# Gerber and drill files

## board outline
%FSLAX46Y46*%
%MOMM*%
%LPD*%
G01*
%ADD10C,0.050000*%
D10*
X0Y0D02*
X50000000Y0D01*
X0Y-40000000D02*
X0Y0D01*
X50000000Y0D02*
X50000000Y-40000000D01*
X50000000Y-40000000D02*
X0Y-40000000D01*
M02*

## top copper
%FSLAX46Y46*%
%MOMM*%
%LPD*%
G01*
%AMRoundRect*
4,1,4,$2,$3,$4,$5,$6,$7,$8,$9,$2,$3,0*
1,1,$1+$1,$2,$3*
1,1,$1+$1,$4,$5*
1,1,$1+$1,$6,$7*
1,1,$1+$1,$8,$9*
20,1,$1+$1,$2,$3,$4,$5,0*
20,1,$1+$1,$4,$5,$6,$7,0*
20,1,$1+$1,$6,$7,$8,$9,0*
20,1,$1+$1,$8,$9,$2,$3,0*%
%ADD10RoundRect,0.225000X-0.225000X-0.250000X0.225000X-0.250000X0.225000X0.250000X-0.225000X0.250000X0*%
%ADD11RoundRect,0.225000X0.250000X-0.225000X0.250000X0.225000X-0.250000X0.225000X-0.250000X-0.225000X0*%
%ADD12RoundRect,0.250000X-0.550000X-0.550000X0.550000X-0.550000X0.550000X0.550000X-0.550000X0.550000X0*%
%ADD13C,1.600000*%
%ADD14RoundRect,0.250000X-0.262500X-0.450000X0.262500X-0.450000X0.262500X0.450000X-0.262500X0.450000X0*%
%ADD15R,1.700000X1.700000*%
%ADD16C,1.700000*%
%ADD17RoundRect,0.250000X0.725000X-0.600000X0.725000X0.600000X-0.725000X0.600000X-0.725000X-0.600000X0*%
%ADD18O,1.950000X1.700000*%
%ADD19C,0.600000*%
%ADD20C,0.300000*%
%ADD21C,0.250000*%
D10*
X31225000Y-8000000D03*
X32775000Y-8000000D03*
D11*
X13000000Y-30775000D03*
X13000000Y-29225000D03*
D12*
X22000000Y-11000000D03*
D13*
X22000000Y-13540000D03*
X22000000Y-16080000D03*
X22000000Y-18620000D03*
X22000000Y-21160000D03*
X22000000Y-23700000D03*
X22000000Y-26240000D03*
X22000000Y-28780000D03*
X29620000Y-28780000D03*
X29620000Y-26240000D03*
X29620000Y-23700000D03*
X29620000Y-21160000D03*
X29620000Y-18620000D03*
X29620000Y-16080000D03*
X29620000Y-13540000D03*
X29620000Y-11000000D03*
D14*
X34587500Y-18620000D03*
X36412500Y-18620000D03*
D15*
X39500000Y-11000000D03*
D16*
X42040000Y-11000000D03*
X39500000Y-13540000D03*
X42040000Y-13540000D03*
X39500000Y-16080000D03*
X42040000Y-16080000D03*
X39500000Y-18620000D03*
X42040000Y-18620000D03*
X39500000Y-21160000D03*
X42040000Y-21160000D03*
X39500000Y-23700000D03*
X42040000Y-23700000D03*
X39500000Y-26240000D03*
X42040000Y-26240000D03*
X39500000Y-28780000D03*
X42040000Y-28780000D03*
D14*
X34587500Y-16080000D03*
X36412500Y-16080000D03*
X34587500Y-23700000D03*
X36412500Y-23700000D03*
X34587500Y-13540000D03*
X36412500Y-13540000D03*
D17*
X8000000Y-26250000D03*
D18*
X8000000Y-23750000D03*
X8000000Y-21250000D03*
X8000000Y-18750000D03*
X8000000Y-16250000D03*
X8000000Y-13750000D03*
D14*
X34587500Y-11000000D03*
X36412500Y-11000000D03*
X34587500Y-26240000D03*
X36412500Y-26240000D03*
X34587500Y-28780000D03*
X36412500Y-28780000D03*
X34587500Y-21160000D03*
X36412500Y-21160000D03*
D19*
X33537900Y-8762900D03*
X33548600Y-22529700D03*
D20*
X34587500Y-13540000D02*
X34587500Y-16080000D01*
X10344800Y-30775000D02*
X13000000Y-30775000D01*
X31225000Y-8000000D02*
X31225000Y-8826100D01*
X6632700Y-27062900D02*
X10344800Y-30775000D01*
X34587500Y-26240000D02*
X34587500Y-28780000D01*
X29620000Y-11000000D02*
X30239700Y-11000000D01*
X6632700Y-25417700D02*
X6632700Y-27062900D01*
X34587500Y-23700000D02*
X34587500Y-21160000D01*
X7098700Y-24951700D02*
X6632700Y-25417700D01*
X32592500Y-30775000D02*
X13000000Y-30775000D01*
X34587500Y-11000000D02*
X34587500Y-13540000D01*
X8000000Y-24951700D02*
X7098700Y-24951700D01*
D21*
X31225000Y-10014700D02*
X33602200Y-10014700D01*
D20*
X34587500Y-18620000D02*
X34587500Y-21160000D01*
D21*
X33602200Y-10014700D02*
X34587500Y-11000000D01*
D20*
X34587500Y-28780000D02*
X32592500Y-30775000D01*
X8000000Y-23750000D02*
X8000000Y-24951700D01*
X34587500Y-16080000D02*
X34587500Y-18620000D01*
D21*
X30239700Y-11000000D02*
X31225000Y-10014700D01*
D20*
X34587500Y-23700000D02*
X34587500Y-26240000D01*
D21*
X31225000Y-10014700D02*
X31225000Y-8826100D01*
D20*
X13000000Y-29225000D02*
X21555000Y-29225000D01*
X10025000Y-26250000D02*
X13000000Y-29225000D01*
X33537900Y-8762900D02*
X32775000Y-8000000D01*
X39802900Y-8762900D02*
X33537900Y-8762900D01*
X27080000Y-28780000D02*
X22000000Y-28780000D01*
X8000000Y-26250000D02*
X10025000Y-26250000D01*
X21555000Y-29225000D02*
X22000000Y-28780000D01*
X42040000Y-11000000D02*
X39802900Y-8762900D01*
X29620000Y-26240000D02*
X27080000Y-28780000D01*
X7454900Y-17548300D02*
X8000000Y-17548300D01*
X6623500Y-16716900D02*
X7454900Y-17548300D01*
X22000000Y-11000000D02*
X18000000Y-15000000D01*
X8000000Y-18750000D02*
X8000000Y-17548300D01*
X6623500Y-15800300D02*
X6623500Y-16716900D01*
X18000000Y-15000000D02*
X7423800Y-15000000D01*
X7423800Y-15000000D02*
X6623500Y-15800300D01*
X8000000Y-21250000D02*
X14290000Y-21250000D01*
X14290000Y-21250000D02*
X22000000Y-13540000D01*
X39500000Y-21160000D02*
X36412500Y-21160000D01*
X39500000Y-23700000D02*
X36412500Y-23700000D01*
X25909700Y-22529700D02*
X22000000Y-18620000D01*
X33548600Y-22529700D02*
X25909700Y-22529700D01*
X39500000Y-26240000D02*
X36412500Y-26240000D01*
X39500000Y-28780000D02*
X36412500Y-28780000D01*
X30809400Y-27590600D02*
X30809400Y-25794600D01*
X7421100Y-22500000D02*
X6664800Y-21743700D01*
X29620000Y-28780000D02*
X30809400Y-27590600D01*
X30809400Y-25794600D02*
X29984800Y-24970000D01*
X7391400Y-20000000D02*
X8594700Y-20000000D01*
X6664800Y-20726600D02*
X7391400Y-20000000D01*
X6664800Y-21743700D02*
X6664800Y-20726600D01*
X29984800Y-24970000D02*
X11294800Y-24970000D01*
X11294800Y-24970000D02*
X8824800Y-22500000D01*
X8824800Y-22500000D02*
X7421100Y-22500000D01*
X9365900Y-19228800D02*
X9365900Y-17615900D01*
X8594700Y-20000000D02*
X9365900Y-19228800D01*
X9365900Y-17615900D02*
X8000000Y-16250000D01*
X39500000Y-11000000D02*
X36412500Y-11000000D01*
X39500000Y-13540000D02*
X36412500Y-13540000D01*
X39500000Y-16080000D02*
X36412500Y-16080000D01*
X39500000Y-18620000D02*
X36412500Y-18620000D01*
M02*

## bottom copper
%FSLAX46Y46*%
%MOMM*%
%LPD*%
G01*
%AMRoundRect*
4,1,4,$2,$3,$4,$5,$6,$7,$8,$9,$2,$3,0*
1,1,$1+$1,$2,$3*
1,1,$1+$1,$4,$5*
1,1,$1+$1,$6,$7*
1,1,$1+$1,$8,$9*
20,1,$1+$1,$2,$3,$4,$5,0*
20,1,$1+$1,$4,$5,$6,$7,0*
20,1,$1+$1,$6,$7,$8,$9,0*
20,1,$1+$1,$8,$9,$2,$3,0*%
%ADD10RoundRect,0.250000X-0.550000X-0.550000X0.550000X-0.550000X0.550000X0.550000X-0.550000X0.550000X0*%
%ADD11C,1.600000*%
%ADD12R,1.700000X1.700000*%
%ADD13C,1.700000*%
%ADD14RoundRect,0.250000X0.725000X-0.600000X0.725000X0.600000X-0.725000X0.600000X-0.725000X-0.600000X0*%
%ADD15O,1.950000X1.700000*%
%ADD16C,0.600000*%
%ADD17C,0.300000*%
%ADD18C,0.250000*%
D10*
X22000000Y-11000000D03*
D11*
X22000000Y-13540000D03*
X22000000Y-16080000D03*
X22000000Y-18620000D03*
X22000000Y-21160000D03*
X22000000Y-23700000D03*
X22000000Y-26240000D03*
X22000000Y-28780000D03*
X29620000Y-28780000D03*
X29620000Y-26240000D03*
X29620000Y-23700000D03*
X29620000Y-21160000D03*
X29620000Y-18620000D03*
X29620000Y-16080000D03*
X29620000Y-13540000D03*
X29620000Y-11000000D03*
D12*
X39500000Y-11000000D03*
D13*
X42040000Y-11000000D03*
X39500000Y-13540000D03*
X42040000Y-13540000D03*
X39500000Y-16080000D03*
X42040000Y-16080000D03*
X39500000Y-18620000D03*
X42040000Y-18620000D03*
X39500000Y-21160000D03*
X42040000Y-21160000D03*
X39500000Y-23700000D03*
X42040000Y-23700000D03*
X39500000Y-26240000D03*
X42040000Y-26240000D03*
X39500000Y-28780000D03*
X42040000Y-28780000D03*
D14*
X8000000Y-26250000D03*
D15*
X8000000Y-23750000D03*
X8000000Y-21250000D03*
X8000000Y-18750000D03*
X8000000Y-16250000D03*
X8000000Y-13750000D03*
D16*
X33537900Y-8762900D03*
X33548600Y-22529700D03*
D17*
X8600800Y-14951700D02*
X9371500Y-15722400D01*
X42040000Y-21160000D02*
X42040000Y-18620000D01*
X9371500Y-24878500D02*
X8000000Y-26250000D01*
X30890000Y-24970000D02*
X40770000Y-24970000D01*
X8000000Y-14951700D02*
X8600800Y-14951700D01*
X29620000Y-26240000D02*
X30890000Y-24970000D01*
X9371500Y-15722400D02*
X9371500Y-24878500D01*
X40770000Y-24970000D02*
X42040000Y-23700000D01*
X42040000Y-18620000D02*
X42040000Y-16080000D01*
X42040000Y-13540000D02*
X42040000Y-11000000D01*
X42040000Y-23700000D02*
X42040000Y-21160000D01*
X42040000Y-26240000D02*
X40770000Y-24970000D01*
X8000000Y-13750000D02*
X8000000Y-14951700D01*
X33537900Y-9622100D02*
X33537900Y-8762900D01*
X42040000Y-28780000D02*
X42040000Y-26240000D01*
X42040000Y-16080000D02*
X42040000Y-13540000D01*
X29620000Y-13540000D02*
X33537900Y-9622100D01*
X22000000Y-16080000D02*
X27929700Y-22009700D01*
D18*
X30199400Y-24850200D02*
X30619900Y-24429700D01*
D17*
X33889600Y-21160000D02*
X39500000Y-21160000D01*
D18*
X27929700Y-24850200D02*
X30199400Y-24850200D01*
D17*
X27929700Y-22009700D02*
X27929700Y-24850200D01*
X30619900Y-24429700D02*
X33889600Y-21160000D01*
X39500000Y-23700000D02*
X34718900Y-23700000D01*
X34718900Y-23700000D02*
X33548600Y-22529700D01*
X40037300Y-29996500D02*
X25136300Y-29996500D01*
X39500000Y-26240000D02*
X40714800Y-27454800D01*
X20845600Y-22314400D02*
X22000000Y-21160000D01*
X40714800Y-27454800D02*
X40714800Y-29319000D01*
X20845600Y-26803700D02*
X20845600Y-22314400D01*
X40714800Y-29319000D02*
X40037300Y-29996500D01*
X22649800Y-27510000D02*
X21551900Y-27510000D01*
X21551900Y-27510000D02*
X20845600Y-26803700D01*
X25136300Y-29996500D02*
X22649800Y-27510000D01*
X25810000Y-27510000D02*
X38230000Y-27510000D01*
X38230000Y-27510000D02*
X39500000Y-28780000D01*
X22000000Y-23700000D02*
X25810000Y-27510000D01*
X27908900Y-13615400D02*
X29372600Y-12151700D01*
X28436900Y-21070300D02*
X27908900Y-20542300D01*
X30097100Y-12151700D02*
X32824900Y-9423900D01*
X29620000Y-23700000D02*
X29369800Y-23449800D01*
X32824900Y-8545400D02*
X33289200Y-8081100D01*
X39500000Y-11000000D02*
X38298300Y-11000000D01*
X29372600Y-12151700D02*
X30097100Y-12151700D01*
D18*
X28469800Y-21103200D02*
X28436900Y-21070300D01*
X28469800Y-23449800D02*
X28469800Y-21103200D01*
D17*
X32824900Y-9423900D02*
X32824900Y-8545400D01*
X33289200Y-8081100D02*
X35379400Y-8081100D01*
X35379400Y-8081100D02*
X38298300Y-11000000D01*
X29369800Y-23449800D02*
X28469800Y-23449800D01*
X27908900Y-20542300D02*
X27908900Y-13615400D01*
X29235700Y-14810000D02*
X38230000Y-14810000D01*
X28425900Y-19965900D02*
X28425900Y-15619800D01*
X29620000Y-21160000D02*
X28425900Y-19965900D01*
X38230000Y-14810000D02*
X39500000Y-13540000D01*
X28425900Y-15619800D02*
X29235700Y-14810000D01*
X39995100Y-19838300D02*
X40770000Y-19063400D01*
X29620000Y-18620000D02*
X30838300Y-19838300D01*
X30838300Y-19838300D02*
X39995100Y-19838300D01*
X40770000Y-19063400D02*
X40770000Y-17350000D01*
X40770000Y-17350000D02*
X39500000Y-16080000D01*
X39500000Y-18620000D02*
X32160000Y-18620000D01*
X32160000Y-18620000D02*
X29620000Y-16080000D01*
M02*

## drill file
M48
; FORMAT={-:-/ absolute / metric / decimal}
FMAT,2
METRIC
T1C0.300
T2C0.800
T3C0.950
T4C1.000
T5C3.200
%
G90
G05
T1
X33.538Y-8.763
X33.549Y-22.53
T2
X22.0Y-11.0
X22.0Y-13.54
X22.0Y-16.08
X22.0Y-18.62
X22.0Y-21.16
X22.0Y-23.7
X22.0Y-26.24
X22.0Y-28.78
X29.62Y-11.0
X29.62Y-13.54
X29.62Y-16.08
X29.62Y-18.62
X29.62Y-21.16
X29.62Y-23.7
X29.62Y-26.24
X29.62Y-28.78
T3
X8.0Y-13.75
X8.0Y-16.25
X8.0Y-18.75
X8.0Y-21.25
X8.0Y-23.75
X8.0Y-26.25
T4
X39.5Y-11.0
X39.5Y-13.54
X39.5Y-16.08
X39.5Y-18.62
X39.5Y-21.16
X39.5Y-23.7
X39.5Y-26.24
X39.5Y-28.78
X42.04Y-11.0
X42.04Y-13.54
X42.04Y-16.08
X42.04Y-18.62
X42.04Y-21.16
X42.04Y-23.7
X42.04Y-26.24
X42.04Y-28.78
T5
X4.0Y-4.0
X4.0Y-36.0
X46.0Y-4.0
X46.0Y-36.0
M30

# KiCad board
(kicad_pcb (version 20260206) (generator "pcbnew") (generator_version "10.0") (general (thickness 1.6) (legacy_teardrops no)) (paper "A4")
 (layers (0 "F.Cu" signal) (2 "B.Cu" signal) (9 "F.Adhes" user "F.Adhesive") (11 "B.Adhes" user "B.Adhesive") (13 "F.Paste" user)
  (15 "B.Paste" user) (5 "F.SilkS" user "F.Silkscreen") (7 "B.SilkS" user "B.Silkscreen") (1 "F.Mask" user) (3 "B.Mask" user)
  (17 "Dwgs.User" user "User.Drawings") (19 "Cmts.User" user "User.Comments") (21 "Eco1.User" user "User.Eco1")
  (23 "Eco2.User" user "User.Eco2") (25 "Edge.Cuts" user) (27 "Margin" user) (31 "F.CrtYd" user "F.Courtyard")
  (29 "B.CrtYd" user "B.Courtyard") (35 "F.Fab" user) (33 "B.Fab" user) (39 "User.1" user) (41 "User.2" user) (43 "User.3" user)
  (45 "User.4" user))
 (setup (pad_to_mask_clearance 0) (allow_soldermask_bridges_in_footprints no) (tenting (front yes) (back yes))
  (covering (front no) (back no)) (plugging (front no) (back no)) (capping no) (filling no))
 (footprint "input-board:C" (layer "F.Cu") (at 32 8)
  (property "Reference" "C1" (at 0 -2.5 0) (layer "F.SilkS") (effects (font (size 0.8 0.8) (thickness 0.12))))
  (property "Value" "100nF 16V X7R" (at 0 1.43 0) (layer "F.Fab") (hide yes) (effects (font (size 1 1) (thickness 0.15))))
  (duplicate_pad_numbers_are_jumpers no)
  (pad "1" smd roundrect (at -0.775 0) (size 0.9 0.95) (layers "F.Cu" "F.Mask" "F.Paste") (roundrect_rratio 0.25) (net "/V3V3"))
  (pad "2" smd roundrect (at 0.775 0) (size 0.9 0.95) (layers "F.Cu" "F.Mask" "F.Paste") (roundrect_rratio 0.25) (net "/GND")))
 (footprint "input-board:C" (layer "F.Cu") (at 13 30 90)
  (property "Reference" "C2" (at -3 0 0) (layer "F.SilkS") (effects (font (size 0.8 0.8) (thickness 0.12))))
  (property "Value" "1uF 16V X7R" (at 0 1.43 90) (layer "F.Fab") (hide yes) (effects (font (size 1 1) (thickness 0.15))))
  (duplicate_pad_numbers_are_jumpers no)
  (pad "1" smd roundrect (at -0.775 0 90) (size 0.9 0.95) (layers "F.Cu" "F.Mask" "F.Paste") (roundrect_rratio 0.25) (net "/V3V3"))
  (pad "2" smd roundrect (at 0.775 0 90) (size 0.9 0.95) (layers "F.Cu" "F.Mask" "F.Paste") (roundrect_rratio 0.25) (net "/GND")))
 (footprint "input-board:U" (layer "F.Cu") (at 22 11)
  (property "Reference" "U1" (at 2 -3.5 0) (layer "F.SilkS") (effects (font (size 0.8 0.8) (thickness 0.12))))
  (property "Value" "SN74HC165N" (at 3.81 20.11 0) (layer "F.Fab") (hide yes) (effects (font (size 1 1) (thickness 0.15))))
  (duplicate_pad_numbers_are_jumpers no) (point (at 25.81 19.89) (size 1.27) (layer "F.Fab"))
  (pad "1" thru_hole roundrect (at 0 0) (size 1.6 1.6) (drill 0.8) (layers "*.Cu" "*.Mask") (remove_unused_layers no)
   (roundrect_rratio 0.15625) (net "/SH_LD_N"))
  (pad "2" thru_hole circle (at 0 2.54) (size 1.6 1.6) (drill 0.8) (layers "*.Cu" "*.Mask") (remove_unused_layers no) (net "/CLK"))
  (pad "3" thru_hole circle (at 0 5.08) (size 1.6 1.6) (drill 0.8) (layers "*.Cu" "*.Mask") (remove_unused_layers no) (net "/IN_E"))
  (pad "4" thru_hole circle (at 0 7.62) (size 1.6 1.6) (drill 0.8) (layers "*.Cu" "*.Mask") (remove_unused_layers no) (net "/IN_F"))
  (pad "5" thru_hole circle (at 0 10.16) (size 1.6 1.6) (drill 0.8) (layers "*.Cu" "*.Mask") (remove_unused_layers no) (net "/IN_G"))
  (pad "6" thru_hole circle (at 0 12.7) (size 1.6 1.6) (drill 0.8) (layers "*.Cu" "*.Mask") (remove_unused_layers no) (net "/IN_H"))
  (pad "7" thru_hole circle (at 0 15.24) (size 1.6 1.6) (drill 0.8) (layers "*.Cu" "*.Mask") (remove_unused_layers no)
   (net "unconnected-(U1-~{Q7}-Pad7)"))
  (pad "8" thru_hole circle (at 0 17.78) (size 1.6 1.6) (drill 0.8) (layers "*.Cu" "*.Mask") (remove_unused_layers no) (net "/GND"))
  (pad "9" thru_hole circle (at 7.62 17.78) (size 1.6 1.6) (drill 0.8) (layers "*.Cu" "*.Mask") (remove_unused_layers no) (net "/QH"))
  (pad "10" thru_hole circle (at 7.62 15.24) (size 1.6 1.6) (drill 0.8) (layers "*.Cu" "*.Mask") (remove_unused_layers no) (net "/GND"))
  (pad "11" thru_hole circle (at 7.62 12.7) (size 1.6 1.6) (drill 0.8) (layers "*.Cu" "*.Mask") (remove_unused_layers no) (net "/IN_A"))
  (pad "12" thru_hole circle (at 7.62 10.16) (size 1.6 1.6) (drill 0.8) (layers "*.Cu" "*.Mask") (remove_unused_layers no) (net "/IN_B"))
  (pad "13" thru_hole circle (at 7.62 7.62) (size 1.6 1.6) (drill 0.8) (layers "*.Cu" "*.Mask") (remove_unused_layers no) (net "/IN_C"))
  (pad "14" thru_hole circle (at 7.62 5.08) (size 1.6 1.6) (drill 0.8) (layers "*.Cu" "*.Mask") (remove_unused_layers no) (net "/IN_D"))
  (pad "15" thru_hole circle (at 7.62 2.54) (size 1.6 1.6) (drill 0.8) (layers "*.Cu" "*.Mask") (remove_unused_layers no) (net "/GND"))
  (pad "16" thru_hole circle (at 7.62 0) (size 1.6 1.6) (drill 0.8) (layers "*.Cu" "*.Mask") (remove_unused_layers no) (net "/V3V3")))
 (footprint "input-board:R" (layer "F.Cu") (at 35.5 18.62)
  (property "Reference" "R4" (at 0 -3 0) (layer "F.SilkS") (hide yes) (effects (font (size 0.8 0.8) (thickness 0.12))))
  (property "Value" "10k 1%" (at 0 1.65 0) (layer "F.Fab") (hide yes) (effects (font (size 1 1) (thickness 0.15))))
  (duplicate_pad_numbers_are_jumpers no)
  (pad "1" smd roundrect (at -0.9125 0) (size 1.025 1.4) (layers "F.Cu" "F.Mask" "F.Paste") (roundrect_rratio 0.243902) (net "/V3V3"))
  (pad "2" smd roundrect (at 0.9125 0) (size 1.025 1.4) (layers "F.Cu" "F.Mask" "F.Paste") (roundrect_rratio 0.243902) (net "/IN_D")))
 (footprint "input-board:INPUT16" (layer "F.Cu") (at 39.5 11)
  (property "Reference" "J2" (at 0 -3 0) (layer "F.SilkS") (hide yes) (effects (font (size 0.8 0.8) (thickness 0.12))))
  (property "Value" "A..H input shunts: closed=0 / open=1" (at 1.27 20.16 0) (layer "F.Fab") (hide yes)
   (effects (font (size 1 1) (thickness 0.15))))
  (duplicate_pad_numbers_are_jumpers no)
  (pad "1" thru_hole rect (at 0 0) (size 1.7 1.7) (drill 1) (layers "*.Cu" "*.Mask") (remove_unused_layers no) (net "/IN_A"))
  (pad "2" thru_hole circle (at 2.54 0) (size 1.7 1.7) (drill 1) (layers "*.Cu" "*.Mask") (remove_unused_layers no) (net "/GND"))
  (pad "3" thru_hole circle (at 0 2.54) (size 1.7 1.7) (drill 1) (layers "*.Cu" "*.Mask") (remove_unused_layers no) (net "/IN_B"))
  (pad "4" thru_hole circle (at 2.54 2.54) (size 1.7 1.7) (drill 1) (layers "*.Cu" "*.Mask") (remove_unused_layers no) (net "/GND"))
  (pad "5" thru_hole circle (at 0 5.08) (size 1.7 1.7) (drill 1) (layers "*.Cu" "*.Mask") (remove_unused_layers no) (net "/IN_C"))
  (pad "6" thru_hole circle (at 2.54 5.08) (size 1.7 1.7) (drill 1) (layers "*.Cu" "*.Mask") (remove_unused_layers no) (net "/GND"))
  (pad "7" thru_hole circle (at 0 7.62) (size 1.7 1.7) (drill 1) (layers "*.Cu" "*.Mask") (remove_unused_layers no) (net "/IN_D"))
  (pad "8" thru_hole circle (at 2.54 7.62) (size 1.7 1.7) (drill 1) (layers "*.Cu" "*.Mask") (remove_unused_layers no) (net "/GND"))
  (pad "9" thru_hole circle (at 0 10.16) (size 1.7 1.7) (drill 1) (layers "*.Cu" "*.Mask") (remove_unused_layers no) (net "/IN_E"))
  (pad "10" thru_hole circle (at 2.54 10.16) (size 1.7 1.7) (drill 1) (layers "*.Cu" "*.Mask") (remove_unused_layers no) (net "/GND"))
  (pad "11" thru_hole circle (at 0 12.7) (size 1.7 1.7) (drill 1) (layers "*.Cu" "*.Mask") (remove_unused_layers no) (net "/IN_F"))
  (pad "12" thru_hole circle (at 2.54 12.7) (size 1.7 1.7) (drill 1) (layers "*.Cu" "*.Mask") (remove_unused_layers no) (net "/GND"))
  (pad "13" thru_hole circle (at 0 15.24) (size 1.7 1.7) (drill 1) (layers "*.Cu" "*.Mask") (remove_unused_layers no) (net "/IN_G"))
  (pad "14" thru_hole circle (at 2.54 15.24) (size 1.7 1.7) (drill 1) (layers "*.Cu" "*.Mask") (remove_unused_layers no) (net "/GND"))
  (pad "15" thru_hole circle (at 0 17.78) (size 1.7 1.7) (drill 1) (layers "*.Cu" "*.Mask") (remove_unused_layers no) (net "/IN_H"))
  (pad "16" thru_hole circle (at 2.54 17.78) (size 1.7 1.7) (drill 1) (layers "*.Cu" "*.Mask") (remove_unused_layers no) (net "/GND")))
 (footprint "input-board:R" (layer "F.Cu") (at 35.5 16.08)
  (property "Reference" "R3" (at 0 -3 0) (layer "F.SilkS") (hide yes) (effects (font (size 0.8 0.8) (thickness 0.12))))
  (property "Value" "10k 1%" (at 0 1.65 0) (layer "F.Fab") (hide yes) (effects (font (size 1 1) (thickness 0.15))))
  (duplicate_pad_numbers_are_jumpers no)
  (pad "1" smd roundrect (at -0.9125 0) (size 1.025 1.4) (layers "F.Cu" "F.Mask" "F.Paste") (roundrect_rratio 0.243902) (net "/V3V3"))
  (pad "2" smd roundrect (at 0.9125 0) (size 1.025 1.4) (layers "F.Cu" "F.Mask" "F.Paste") (roundrect_rratio 0.243902) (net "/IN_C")))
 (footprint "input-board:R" (layer "F.Cu") (at 35.5 23.7)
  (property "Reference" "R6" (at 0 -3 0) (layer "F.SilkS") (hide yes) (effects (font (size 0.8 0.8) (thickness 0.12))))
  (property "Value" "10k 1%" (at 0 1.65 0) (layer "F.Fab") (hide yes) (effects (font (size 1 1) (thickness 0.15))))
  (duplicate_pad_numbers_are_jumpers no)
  (pad "1" smd roundrect (at -0.9125 0) (size 1.025 1.4) (layers "F.Cu" "F.Mask" "F.Paste") (roundrect_rratio 0.243902) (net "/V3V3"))
  (pad "2" smd roundrect (at 0.9125 0) (size 1.025 1.4) (layers "F.Cu" "F.Mask" "F.Paste") (roundrect_rratio 0.243902) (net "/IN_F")))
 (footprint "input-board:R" (layer "F.Cu") (at 35.5 13.54)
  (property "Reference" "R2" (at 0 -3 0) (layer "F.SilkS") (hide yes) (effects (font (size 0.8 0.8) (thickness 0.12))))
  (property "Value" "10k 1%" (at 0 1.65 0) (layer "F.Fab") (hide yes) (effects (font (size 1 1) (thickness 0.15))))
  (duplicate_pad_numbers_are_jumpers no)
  (pad "1" smd roundrect (at -0.9125 0) (size 1.025 1.4) (layers "F.Cu" "F.Mask" "F.Paste") (roundrect_rratio 0.243902) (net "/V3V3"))
  (pad "2" smd roundrect (at 0.9125 0) (size 1.025 1.4) (layers "F.Cu" "F.Mask" "F.Paste") (roundrect_rratio 0.243902) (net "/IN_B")))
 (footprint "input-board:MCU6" (layer "F.Cu") (at 8 26.25 90)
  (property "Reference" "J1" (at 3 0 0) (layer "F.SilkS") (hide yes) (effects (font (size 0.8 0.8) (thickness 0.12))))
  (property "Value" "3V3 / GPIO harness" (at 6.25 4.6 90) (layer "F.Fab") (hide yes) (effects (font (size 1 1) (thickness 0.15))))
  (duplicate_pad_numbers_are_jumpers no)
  (pad "1" thru_hole roundrect (at 0 0 90) (size 1.7 1.95) (drill 0.95) (layers "*.Cu" "*.Mask") (remove_unused_layers no)
   (roundrect_rratio 0.147059) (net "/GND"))
  (pad "2" thru_hole oval (at 2.5 0 90) (size 1.7 1.95) (drill 0.95) (layers "*.Cu" "*.Mask") (remove_unused_layers no) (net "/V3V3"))
  (pad "3" thru_hole oval (at 5 0 90) (size 1.7 1.95) (drill 0.95) (layers "*.Cu" "*.Mask") (remove_unused_layers no) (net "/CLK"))
  (pad "4" thru_hole oval (at 7.5 0 90) (size 1.7 1.95) (drill 0.95) (layers "*.Cu" "*.Mask") (remove_unused_layers no) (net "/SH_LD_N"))
  (pad "5" thru_hole oval (at 10 0 90) (size 1.7 1.95) (drill 0.95) (layers "*.Cu" "*.Mask") (remove_unused_layers no) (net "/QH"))
  (pad "6" thru_hole oval (at 12.5 0 90) (size 1.7 1.95) (drill 0.95) (layers "*.Cu" "*.Mask") (remove_unused_layers no) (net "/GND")))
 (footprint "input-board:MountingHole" (layer "F.Cu") (at 4 36)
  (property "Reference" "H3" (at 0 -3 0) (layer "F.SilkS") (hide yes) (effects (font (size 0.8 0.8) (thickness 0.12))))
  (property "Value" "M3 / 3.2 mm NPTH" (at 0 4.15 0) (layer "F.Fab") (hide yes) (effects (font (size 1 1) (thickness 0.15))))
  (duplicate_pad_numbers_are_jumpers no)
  (pad "" np_thru_hole circle (at 0 0) (size 3.2 3.2) (drill 3.2) (layers "*.Cu" "*.Mask")))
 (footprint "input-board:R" (layer "F.Cu") (at 35.5 11)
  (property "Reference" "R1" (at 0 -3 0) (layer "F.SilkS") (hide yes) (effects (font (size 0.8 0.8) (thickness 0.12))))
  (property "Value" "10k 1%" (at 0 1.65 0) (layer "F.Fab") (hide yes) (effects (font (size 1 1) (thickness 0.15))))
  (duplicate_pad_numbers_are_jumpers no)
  (pad "1" smd roundrect (at -0.9125 0) (size 1.025 1.4) (layers "F.Cu" "F.Mask" "F.Paste") (roundrect_rratio 0.243902) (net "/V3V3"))
  (pad "2" smd roundrect (at 0.9125 0) (size 1.025 1.4) (layers "F.Cu" "F.Mask" "F.Paste") (roundrect_rratio 0.243902) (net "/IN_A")))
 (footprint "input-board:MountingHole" (layer "F.Cu") (at 4 4)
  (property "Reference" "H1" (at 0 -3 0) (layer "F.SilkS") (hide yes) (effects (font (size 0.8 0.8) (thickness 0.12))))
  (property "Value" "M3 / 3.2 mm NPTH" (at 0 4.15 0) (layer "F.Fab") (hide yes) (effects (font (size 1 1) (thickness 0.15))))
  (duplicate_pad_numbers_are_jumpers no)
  (pad "" np_thru_hole circle (at 0 0) (size 3.2 3.2) (drill 3.2) (layers "*.Cu" "*.Mask")))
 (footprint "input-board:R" (layer "F.Cu") (at 35.5 26.24)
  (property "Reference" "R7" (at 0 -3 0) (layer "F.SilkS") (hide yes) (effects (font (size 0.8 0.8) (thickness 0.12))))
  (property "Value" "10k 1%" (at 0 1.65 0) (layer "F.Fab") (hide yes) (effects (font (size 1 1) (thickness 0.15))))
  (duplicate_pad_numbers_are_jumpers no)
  (pad "1" smd roundrect (at -0.9125 0) (size 1.025 1.4) (layers "F.Cu" "F.Mask" "F.Paste") (roundrect_rratio 0.243902) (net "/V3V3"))
  (pad "2" smd roundrect (at 0.9125 0) (size 1.025 1.4) (layers "F.Cu" "F.Mask" "F.Paste") (roundrect_rratio 0.243902) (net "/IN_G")))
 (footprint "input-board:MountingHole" (layer "F.Cu") (at 46 36)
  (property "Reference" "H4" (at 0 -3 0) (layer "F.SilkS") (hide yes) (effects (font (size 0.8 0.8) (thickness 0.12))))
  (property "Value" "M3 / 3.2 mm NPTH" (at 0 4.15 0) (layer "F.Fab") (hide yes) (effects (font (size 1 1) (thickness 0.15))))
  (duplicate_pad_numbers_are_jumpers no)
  (pad "" np_thru_hole circle (at 0 0) (size 3.2 3.2) (drill 3.2) (layers "*.Cu" "*.Mask")))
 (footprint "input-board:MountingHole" (layer "F.Cu") (at 46 4)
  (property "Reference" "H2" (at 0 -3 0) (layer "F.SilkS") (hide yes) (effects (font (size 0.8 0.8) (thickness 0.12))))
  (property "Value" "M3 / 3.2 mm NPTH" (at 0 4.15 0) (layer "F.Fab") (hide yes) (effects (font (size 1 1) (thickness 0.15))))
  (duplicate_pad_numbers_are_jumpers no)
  (pad "" np_thru_hole circle (at 0 0) (size 3.2 3.2) (drill 3.2) (layers "*.Cu" "*.Mask")))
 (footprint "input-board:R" (layer "F.Cu") (at 35.5 28.78)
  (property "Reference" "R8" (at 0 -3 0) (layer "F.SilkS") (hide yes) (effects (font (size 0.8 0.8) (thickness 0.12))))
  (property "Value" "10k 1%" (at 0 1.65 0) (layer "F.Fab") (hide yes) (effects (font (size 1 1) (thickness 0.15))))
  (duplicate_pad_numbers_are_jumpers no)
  (pad "1" smd roundrect (at -0.9125 0) (size 1.025 1.4) (layers "F.Cu" "F.Mask" "F.Paste") (roundrect_rratio 0.243902) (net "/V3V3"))
  (pad "2" smd roundrect (at 0.9125 0) (size 1.025 1.4) (layers "F.Cu" "F.Mask" "F.Paste") (roundrect_rratio 0.243902) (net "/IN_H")))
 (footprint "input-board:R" (layer "F.Cu") (at 35.5 21.16)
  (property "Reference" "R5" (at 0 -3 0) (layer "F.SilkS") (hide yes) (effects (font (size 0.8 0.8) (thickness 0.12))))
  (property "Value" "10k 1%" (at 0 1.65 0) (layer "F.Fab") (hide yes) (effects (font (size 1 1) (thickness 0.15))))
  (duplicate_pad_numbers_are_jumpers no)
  (pad "1" smd roundrect (at -0.9125 0) (size 1.025 1.4) (layers "F.Cu" "F.Mask" "F.Paste") (roundrect_rratio 0.243902) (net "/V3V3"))
  (pad "2" smd roundrect (at 0.9125 0) (size 1.025 1.4) (layers "F.Cu" "F.Mask" "F.Paste") (roundrect_rratio 0.243902) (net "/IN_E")))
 (gr_line (start 0 0) (end 50 0) (stroke (width 0.05) (type default)) (layer "Edge.Cuts"))
 (gr_line (start 0 40) (end 0 0) (stroke (width 0.05) (type default)) (layer "Edge.Cuts"))
 (gr_line (start 50 0) (end 50 40) (stroke (width 0.05) (type default)) (layer "Edge.Cuts"))
 (gr_line (start 50 40) (end 0 40) (stroke (width 0.05) (type default)) (layer "Edge.Cuts"))
 (segment (start 34.5875 13.54) (end 34.5875 16.08) (width 0.3) (layer "F.Cu") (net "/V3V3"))
 (segment (start 10.3448 30.775) (end 13 30.775) (width 0.3) (layer "F.Cu") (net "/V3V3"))
 (segment (start 31.225 8) (end 31.225 8.8261) (width 0.3) (layer "F.Cu") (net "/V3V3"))
 (segment (start 6.6327 27.0629) (end 10.3448 30.775) (width 0.3) (layer "F.Cu") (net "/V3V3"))
 (segment (start 34.5875 26.24) (end 34.5875 28.78) (width 0.3) (layer "F.Cu") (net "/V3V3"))
 (segment (start 29.62 11) (end 30.2397 11) (width 0.3) (layer "F.Cu") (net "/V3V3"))
 (segment (start 6.6327 25.4177) (end 6.6327 27.0629) (width 0.3) (layer "F.Cu") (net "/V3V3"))
 (segment (start 34.5875 23.7) (end 34.5875 21.16) (width 0.3) (layer "F.Cu") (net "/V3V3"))
 (segment (start 7.0987 24.9517) (end 6.6327 25.4177) (width 0.3) (layer "F.Cu") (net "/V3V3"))
 (segment (start 32.5925 30.775) (end 13 30.775) (width 0.3) (layer "F.Cu") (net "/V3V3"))
 (segment (start 34.5875 11) (end 34.5875 13.54) (width 0.3) (layer "F.Cu") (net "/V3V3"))
 (segment (start 8 24.9517) (end 7.0987 24.9517) (width 0.3) (layer "F.Cu") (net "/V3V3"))
 (segment (start 31.225 10.0147) (end 33.6022 10.0147) (width 0.25) (layer "F.Cu") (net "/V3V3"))
 (segment (start 34.5875 18.62) (end 34.5875 21.16) (width 0.3) (layer "F.Cu") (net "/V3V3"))
 (segment (start 33.6022 10.0147) (end 34.5875 11) (width 0.25) (layer "F.Cu") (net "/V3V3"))
 (segment (start 34.5875 28.78) (end 32.5925 30.775) (width 0.3) (layer "F.Cu") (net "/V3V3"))
 (segment (start 8 23.75) (end 8 24.9517) (width 0.3) (layer "F.Cu") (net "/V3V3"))
 (segment (start 34.5875 16.08) (end 34.5875 18.62) (width 0.3) (layer "F.Cu") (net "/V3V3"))
 (segment (start 30.2397 11) (end 31.225 10.0147) (width 0.25) (layer "F.Cu") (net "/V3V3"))
 (segment (start 34.5875 23.7) (end 34.5875 26.24) (width 0.3) (layer "F.Cu") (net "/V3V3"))
 (segment (start 31.225 10.0147) (end 31.225 8.8261) (width 0.25) (layer "F.Cu") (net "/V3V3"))
 (segment (start 13 29.225) (end 21.555 29.225) (width 0.3) (layer "F.Cu") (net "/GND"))
 (segment (start 10.025 26.25) (end 13 29.225) (width 0.3) (layer "F.Cu") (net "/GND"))
 (segment (start 33.5379 8.7629) (end 32.775 8) (width 0.3) (layer "F.Cu") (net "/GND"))
 (segment (start 39.8029 8.7629) (end 33.5379 8.7629) (width 0.3) (layer "F.Cu") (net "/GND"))
 (segment (start 27.08 28.78) (end 22 28.78) (width 0.3) (layer "F.Cu") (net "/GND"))
 (segment (start 8 26.25) (end 10.025 26.25) (width 0.3) (layer "F.Cu") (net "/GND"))
 (segment (start 21.555 29.225) (end 22 28.78) (width 0.3) (layer "F.Cu") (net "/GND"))
 (segment (start 42.04 11) (end 39.8029 8.7629) (width 0.3) (layer "F.Cu") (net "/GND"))
 (segment (start 29.62 26.24) (end 27.08 28.78) (width 0.3) (layer "F.Cu") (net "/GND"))
 (via (at 33.5379 8.7629) (size 0.6) (drill 0.3) (layers "F.Cu" "B.Cu") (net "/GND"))
 (segment (start 8.6008 14.9517) (end 9.3715 15.7224) (width 0.3) (layer "B.Cu") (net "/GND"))
 (segment (start 42.04 21.16) (end 42.04 18.62) (width 0.3) (layer "B.Cu") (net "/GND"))
 (segment (start 9.3715 24.8785) (end 8 26.25) (width 0.3) (layer "B.Cu") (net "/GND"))
 (segment (start 30.89 24.97) (end 40.77 24.97) (width 0.3) (layer "B.Cu") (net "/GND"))
 (segment (start 8 14.9517) (end 8.6008 14.9517) (width 0.3) (layer "B.Cu") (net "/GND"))
 (segment (start 29.62 26.24) (end 30.89 24.97) (width 0.3) (layer "B.Cu") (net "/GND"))
 (segment (start 9.3715 15.7224) (end 9.3715 24.8785) (width 0.3) (layer "B.Cu") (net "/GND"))
 (segment (start 40.77 24.97) (end 42.04 23.7) (width 0.3) (layer "B.Cu") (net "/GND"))
 (segment (start 42.04 18.62) (end 42.04 16.08) (width 0.3) (layer "B.Cu") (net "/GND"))
 (segment (start 42.04 13.54) (end 42.04 11) (width 0.3) (layer "B.Cu") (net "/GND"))
 (segment (start 42.04 23.7) (end 42.04 21.16) (width 0.3) (layer "B.Cu") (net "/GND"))
 (segment (start 42.04 26.24) (end 40.77 24.97) (width 0.3) (layer "B.Cu") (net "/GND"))
 (segment (start 8 13.75) (end 8 14.9517) (width 0.3) (layer "B.Cu") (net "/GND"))
 (segment (start 33.5379 9.6221) (end 33.5379 8.7629) (width 0.3) (layer "B.Cu") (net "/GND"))
 (segment (start 42.04 28.78) (end 42.04 26.24) (width 0.3) (layer "B.Cu") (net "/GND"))
 (segment (start 42.04 16.08) (end 42.04 13.54) (width 0.3) (layer "B.Cu") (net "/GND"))
 (segment (start 29.62 13.54) (end 33.5379 9.6221) (width 0.3) (layer "B.Cu") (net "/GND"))
 (segment (start 7.4549 17.5483) (end 8 17.5483) (width 0.3) (layer "F.Cu") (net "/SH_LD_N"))
 (segment (start 6.6235 16.7169) (end 7.4549 17.5483) (width 0.3) (layer "F.Cu") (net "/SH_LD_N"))
 (segment (start 22 11) (end 18 15) (width 0.3) (layer "F.Cu") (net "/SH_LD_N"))
 (segment (start 8 18.75) (end 8 17.5483) (width 0.3) (layer "F.Cu") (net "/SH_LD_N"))
 (segment (start 6.6235 15.8003) (end 6.6235 16.7169) (width 0.3) (layer "F.Cu") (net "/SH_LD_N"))
 (segment (start 18 15) (end 7.4238 15) (width 0.3) (layer "F.Cu") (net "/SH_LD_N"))
 (segment (start 7.4238 15) (end 6.6235 15.8003) (width 0.3) (layer "F.Cu") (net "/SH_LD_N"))
 (segment (start 8 21.25) (end 14.29 21.25) (width 0.3) (layer "F.Cu") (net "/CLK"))
 (segment (start 14.29 21.25) (end 22 13.54) (width 0.3) (layer "F.Cu") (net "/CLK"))
 (segment (start 39.5 21.16) (end 36.4125 21.16) (width 0.3) (layer "F.Cu") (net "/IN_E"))
 (segment (start 22 16.08) (end 27.9297 22.0097) (width 0.3) (layer "B.Cu") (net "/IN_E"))
 (segment (start 30.1994 24.8502) (end 30.6199 24.4297) (width 0.25) (layer "B.Cu") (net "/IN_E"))
 (segment (start 33.8896 21.16) (end 39.5 21.16) (width 0.3) (layer "B.Cu") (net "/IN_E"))
 (segment (start 27.9297 24.8502) (end 30.1994 24.8502) (width 0.25) (layer "B.Cu") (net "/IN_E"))
 (segment (start 27.9297 22.0097) (end 27.9297 24.8502) (width 0.3) (layer "B.Cu") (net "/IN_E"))
 (segment (start 30.6199 24.4297) (end 33.8896 21.16) (width 0.3) (layer "B.Cu") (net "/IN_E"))
 (segment (start 39.5 23.7) (end 36.4125 23.7) (width 0.3) (layer "F.Cu") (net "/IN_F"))
 (segment (start 25.9097 22.5297) (end 22 18.62) (width 0.3) (layer "F.Cu") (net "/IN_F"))
 (segment (start 33.5486 22.5297) (end 25.9097 22.5297) (width 0.3) (layer "F.Cu") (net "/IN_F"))
 (via (at 33.5486 22.5297) (size 0.6) (drill 0.3) (layers "F.Cu" "B.Cu") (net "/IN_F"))
 (segment (start 39.5 23.7) (end 34.7189 23.7) (width 0.3) (layer "B.Cu") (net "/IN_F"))
 (segment (start 34.7189 23.7) (end 33.5486 22.5297) (width 0.3) (layer "B.Cu") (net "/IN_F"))
 (segment (start 39.5 26.24) (end 36.4125 26.24) (width 0.3) (layer "F.Cu") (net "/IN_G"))
 (segment (start 40.0373 29.9965) (end 25.1363 29.9965) (width 0.3) (layer "B.Cu") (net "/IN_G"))
 (segment (start 39.5 26.24) (end 40.7148 27.4548) (width 0.3) (layer "B.Cu") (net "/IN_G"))
 (segment (start 20.8456 22.3144) (end 22 21.16) (width 0.3) (layer "B.Cu") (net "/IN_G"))
 (segment (start 40.7148 27.4548) (end 40.7148 29.319) (width 0.3) (layer "B.Cu") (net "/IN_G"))
 (segment (start 20.8456 26.8037) (end 20.8456 22.3144) (width 0.3) (layer "B.Cu") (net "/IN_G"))
 (segment (start 40.7148 29.319) (end 40.0373 29.9965) (width 0.3) (layer "B.Cu") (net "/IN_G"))
 (segment (start 22.6498 27.51) (end 21.5519 27.51) (width 0.3) (layer "B.Cu") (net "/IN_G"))
 (segment (start 21.5519 27.51) (end 20.8456 26.8037) (width 0.3) (layer "B.Cu") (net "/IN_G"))
 (segment (start 25.1363 29.9965) (end 22.6498 27.51) (width 0.3) (layer "B.Cu") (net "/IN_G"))
 (segment (start 39.5 28.78) (end 36.4125 28.78) (width 0.3) (layer "F.Cu") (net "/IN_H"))
 (segment (start 25.81 27.51) (end 38.23 27.51) (width 0.3) (layer "B.Cu") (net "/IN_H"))
 (segment (start 38.23 27.51) (end 39.5 28.78) (width 0.3) (layer "B.Cu") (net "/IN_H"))
 (segment (start 22 23.7) (end 25.81 27.51) (width 0.3) (layer "B.Cu") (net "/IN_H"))
 (segment (start 30.8094 27.5906) (end 30.8094 25.7946) (width 0.3) (layer "F.Cu") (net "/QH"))
 (segment (start 7.4211 22.5) (end 6.6648 21.7437) (width 0.3) (layer "F.Cu") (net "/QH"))
 (segment (start 29.62 28.78) (end 30.8094 27.5906) (width 0.3) (layer "F.Cu") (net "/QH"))
 (segment (start 30.8094 25.7946) (end 29.9848 24.97) (width 0.3) (layer "F.Cu") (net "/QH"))
 (segment (start 7.3914 20) (end 8.5947 20) (width 0.3) (layer "F.Cu") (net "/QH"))
 (segment (start 6.6648 20.7266) (end 7.3914 20) (width 0.3) (layer "F.Cu") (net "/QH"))
 (segment (start 6.6648 21.7437) (end 6.6648 20.7266) (width 0.3) (layer "F.Cu") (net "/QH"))
 (segment (start 29.9848 24.97) (end 11.2948 24.97) (width 0.3) (layer "F.Cu") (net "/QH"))
 (segment (start 11.2948 24.97) (end 8.8248 22.5) (width 0.3) (layer "F.Cu") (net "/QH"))
 (segment (start 8.8248 22.5) (end 7.4211 22.5) (width 0.3) (layer "F.Cu") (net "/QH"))
 (segment (start 9.3659 19.2288) (end 9.3659 17.6159) (width 0.3) (layer "F.Cu") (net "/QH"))
 (segment (start 8.5947 20) (end 9.3659 19.2288) (width 0.3) (layer "F.Cu") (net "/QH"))
 (segment (start 9.3659 17.6159) (end 8 16.25) (width 0.3) (layer "F.Cu") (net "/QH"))
 (segment (start 39.5 11) (end 36.4125 11) (width 0.3) (layer "F.Cu") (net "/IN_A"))
 (segment (start 27.9089 13.6154) (end 29.3726 12.1517) (width 0.3) (layer "B.Cu") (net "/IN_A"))
 (segment (start 28.4369 21.0703) (end 27.9089 20.5423) (width 0.3) (layer "B.Cu") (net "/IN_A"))
 (segment (start 30.0971 12.1517) (end 32.8249 9.4239) (width 0.3) (layer "B.Cu") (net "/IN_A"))
 (segment (start 29.62 23.7) (end 29.3698 23.4498) (width 0.3) (layer "B.Cu") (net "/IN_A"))
 (segment (start 32.8249 8.5454) (end 33.2892 8.0811) (width 0.3) (layer "B.Cu") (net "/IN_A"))
 (segment (start 39.5 11) (end 38.2983 11) (width 0.3) (layer "B.Cu") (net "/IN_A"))
 (segment (start 29.3726 12.1517) (end 30.0971 12.1517) (width 0.3) (layer "B.Cu") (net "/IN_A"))
 (segment (start 28.4698 21.1032) (end 28.4369 21.0703) (width 0.25) (layer "B.Cu") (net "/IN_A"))
 (segment (start 28.4698 23.4498) (end 28.4698 21.1032) (width 0.25) (layer "B.Cu") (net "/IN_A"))
 (segment (start 32.8249 9.4239) (end 32.8249 8.5454) (width 0.3) (layer "B.Cu") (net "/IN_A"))
 (segment (start 33.2892 8.0811) (end 35.3794 8.0811) (width 0.3) (layer "B.Cu") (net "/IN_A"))
 (segment (start 35.3794 8.0811) (end 38.2983 11) (width 0.3) (layer "B.Cu") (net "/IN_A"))
 (segment (start 29.3698 23.4498) (end 28.4698 23.4498) (width 0.3) (layer "B.Cu") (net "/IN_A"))
 (segment (start 27.9089 20.5423) (end 27.9089 13.6154) (width 0.3) (layer "B.Cu") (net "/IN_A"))
 (segment (start 39.5 13.54) (end 36.4125 13.54) (width 0.3) (layer "F.Cu") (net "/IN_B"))
 (segment (start 29.2357 14.81) (end 38.23 14.81) (width 0.3) (layer "B.Cu") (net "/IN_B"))
 (segment (start 28.4259 19.9659) (end 28.4259 15.6198) (width 0.3) (layer "B.Cu") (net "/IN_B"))
 (segment (start 29.62 21.16) (end 28.4259 19.9659) (width 0.3) (layer "B.Cu") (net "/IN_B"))
 (segment (start 38.23 14.81) (end 39.5 13.54) (width 0.3) (layer "B.Cu") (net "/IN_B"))
 (segment (start 28.4259 15.6198) (end 29.2357 14.81) (width 0.3) (layer "B.Cu") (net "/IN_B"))
 (segment (start 39.5 16.08) (end 36.4125 16.08) (width 0.3) (layer "F.Cu") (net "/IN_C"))
 (segment (start 39.9951 19.8383) (end 40.77 19.0634) (width 0.3) (layer "B.Cu") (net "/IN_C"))
 (segment (start 29.62 18.62) (end 30.8383 19.8383) (width 0.3) (layer "B.Cu") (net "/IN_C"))
 (segment (start 30.8383 19.8383) (end 39.9951 19.8383) (width 0.3) (layer "B.Cu") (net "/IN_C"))
 (segment (start 40.77 19.0634) (end 40.77 17.35) (width 0.3) (layer "B.Cu") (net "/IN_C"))
 (segment (start 40.77 17.35) (end 39.5 16.08) (width 0.3) (layer "B.Cu") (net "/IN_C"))
 (segment (start 39.5 18.62) (end 36.4125 18.62) (width 0.3) (layer "F.Cu") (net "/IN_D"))
 (segment (start 39.5 18.62) (end 32.16 18.62) (width 0.3) (layer "B.Cu") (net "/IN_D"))
 (segment (start 32.16 18.62) (end 29.62 16.08) (width 0.3) (layer "B.Cu") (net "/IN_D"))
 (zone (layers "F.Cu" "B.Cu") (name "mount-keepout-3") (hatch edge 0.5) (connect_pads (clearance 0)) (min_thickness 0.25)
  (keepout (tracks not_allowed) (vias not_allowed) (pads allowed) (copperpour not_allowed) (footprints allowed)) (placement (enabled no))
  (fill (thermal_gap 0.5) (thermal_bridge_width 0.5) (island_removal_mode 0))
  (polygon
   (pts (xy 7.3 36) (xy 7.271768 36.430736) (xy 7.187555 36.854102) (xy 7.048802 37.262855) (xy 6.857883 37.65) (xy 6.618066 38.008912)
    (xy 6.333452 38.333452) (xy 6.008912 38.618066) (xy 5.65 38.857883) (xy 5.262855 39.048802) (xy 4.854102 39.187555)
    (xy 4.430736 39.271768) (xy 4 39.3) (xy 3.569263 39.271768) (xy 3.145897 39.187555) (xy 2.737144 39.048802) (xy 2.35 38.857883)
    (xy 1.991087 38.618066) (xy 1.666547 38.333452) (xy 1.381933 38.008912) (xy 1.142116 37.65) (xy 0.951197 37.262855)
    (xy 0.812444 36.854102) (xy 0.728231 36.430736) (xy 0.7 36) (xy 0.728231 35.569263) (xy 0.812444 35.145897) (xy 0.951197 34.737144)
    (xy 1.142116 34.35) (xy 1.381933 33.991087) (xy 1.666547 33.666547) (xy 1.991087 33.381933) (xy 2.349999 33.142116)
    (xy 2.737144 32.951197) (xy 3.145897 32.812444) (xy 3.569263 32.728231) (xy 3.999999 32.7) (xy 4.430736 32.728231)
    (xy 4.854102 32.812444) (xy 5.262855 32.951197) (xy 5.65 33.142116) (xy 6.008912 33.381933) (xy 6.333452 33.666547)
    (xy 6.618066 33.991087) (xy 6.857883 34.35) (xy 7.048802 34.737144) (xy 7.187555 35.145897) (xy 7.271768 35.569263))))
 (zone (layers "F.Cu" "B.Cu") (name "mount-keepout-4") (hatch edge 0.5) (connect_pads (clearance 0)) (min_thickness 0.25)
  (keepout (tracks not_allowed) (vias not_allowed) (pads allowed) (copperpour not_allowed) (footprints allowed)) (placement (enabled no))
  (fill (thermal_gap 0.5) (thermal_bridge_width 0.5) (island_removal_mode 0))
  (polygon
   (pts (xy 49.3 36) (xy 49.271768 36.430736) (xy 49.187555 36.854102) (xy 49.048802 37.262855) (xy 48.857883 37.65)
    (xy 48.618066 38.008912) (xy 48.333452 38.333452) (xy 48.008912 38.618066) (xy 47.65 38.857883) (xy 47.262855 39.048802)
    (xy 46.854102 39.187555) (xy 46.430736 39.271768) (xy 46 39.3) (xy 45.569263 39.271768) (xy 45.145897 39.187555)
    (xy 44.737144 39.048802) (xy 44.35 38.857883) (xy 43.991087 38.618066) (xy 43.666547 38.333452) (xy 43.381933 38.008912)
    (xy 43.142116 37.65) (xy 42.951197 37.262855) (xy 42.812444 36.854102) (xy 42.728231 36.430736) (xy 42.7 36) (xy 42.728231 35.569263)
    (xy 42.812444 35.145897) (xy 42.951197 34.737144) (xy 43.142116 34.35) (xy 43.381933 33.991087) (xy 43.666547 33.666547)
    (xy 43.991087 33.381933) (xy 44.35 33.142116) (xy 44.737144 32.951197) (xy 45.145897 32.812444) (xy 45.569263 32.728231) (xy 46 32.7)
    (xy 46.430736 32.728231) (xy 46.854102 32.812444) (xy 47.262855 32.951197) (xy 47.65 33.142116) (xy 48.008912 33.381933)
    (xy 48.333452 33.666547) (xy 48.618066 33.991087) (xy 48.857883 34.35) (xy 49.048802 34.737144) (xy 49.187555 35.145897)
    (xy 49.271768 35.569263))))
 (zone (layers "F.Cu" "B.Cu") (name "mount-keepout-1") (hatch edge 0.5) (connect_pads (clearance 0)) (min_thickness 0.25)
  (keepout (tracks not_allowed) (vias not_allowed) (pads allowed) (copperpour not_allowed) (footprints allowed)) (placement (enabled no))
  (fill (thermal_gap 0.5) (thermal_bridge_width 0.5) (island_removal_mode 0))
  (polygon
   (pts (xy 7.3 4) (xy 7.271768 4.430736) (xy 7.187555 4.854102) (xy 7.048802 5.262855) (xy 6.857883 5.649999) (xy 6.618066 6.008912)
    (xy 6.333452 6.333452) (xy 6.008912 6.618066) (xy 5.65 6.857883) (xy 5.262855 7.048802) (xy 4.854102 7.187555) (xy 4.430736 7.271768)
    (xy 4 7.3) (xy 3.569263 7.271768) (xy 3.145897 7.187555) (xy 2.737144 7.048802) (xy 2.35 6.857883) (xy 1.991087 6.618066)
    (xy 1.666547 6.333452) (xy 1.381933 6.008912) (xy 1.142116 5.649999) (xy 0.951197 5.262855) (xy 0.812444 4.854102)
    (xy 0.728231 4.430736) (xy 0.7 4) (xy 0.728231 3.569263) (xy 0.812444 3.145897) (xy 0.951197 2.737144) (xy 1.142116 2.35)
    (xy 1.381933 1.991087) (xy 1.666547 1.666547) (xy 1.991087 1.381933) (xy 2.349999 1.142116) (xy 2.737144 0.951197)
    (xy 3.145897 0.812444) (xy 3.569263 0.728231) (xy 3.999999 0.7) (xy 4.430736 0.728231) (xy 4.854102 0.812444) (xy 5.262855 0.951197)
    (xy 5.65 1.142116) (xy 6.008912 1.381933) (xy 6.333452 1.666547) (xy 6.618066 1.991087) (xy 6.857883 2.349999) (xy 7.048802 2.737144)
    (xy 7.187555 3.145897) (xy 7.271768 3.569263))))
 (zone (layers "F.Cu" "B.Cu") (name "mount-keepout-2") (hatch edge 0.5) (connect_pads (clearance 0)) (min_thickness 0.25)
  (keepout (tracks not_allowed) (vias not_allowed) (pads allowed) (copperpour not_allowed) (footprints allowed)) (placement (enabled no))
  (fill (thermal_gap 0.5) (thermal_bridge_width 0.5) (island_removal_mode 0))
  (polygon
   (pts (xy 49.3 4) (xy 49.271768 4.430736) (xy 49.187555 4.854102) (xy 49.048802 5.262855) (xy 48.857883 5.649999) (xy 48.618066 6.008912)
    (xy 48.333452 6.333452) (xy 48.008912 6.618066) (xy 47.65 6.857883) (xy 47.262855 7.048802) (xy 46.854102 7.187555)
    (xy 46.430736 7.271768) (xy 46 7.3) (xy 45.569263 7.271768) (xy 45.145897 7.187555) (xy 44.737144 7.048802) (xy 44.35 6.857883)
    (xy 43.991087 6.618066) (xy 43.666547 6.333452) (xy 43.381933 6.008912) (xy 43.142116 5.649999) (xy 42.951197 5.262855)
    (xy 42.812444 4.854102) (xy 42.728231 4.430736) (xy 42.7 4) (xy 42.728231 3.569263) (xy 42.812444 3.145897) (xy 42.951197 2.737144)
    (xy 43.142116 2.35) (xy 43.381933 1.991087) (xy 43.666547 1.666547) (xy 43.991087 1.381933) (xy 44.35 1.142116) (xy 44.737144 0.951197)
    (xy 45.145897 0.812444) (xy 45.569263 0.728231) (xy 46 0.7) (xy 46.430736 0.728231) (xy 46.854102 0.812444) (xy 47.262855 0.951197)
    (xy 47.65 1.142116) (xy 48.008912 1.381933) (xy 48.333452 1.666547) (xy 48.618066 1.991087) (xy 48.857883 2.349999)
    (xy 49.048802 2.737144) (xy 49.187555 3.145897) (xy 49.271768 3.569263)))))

